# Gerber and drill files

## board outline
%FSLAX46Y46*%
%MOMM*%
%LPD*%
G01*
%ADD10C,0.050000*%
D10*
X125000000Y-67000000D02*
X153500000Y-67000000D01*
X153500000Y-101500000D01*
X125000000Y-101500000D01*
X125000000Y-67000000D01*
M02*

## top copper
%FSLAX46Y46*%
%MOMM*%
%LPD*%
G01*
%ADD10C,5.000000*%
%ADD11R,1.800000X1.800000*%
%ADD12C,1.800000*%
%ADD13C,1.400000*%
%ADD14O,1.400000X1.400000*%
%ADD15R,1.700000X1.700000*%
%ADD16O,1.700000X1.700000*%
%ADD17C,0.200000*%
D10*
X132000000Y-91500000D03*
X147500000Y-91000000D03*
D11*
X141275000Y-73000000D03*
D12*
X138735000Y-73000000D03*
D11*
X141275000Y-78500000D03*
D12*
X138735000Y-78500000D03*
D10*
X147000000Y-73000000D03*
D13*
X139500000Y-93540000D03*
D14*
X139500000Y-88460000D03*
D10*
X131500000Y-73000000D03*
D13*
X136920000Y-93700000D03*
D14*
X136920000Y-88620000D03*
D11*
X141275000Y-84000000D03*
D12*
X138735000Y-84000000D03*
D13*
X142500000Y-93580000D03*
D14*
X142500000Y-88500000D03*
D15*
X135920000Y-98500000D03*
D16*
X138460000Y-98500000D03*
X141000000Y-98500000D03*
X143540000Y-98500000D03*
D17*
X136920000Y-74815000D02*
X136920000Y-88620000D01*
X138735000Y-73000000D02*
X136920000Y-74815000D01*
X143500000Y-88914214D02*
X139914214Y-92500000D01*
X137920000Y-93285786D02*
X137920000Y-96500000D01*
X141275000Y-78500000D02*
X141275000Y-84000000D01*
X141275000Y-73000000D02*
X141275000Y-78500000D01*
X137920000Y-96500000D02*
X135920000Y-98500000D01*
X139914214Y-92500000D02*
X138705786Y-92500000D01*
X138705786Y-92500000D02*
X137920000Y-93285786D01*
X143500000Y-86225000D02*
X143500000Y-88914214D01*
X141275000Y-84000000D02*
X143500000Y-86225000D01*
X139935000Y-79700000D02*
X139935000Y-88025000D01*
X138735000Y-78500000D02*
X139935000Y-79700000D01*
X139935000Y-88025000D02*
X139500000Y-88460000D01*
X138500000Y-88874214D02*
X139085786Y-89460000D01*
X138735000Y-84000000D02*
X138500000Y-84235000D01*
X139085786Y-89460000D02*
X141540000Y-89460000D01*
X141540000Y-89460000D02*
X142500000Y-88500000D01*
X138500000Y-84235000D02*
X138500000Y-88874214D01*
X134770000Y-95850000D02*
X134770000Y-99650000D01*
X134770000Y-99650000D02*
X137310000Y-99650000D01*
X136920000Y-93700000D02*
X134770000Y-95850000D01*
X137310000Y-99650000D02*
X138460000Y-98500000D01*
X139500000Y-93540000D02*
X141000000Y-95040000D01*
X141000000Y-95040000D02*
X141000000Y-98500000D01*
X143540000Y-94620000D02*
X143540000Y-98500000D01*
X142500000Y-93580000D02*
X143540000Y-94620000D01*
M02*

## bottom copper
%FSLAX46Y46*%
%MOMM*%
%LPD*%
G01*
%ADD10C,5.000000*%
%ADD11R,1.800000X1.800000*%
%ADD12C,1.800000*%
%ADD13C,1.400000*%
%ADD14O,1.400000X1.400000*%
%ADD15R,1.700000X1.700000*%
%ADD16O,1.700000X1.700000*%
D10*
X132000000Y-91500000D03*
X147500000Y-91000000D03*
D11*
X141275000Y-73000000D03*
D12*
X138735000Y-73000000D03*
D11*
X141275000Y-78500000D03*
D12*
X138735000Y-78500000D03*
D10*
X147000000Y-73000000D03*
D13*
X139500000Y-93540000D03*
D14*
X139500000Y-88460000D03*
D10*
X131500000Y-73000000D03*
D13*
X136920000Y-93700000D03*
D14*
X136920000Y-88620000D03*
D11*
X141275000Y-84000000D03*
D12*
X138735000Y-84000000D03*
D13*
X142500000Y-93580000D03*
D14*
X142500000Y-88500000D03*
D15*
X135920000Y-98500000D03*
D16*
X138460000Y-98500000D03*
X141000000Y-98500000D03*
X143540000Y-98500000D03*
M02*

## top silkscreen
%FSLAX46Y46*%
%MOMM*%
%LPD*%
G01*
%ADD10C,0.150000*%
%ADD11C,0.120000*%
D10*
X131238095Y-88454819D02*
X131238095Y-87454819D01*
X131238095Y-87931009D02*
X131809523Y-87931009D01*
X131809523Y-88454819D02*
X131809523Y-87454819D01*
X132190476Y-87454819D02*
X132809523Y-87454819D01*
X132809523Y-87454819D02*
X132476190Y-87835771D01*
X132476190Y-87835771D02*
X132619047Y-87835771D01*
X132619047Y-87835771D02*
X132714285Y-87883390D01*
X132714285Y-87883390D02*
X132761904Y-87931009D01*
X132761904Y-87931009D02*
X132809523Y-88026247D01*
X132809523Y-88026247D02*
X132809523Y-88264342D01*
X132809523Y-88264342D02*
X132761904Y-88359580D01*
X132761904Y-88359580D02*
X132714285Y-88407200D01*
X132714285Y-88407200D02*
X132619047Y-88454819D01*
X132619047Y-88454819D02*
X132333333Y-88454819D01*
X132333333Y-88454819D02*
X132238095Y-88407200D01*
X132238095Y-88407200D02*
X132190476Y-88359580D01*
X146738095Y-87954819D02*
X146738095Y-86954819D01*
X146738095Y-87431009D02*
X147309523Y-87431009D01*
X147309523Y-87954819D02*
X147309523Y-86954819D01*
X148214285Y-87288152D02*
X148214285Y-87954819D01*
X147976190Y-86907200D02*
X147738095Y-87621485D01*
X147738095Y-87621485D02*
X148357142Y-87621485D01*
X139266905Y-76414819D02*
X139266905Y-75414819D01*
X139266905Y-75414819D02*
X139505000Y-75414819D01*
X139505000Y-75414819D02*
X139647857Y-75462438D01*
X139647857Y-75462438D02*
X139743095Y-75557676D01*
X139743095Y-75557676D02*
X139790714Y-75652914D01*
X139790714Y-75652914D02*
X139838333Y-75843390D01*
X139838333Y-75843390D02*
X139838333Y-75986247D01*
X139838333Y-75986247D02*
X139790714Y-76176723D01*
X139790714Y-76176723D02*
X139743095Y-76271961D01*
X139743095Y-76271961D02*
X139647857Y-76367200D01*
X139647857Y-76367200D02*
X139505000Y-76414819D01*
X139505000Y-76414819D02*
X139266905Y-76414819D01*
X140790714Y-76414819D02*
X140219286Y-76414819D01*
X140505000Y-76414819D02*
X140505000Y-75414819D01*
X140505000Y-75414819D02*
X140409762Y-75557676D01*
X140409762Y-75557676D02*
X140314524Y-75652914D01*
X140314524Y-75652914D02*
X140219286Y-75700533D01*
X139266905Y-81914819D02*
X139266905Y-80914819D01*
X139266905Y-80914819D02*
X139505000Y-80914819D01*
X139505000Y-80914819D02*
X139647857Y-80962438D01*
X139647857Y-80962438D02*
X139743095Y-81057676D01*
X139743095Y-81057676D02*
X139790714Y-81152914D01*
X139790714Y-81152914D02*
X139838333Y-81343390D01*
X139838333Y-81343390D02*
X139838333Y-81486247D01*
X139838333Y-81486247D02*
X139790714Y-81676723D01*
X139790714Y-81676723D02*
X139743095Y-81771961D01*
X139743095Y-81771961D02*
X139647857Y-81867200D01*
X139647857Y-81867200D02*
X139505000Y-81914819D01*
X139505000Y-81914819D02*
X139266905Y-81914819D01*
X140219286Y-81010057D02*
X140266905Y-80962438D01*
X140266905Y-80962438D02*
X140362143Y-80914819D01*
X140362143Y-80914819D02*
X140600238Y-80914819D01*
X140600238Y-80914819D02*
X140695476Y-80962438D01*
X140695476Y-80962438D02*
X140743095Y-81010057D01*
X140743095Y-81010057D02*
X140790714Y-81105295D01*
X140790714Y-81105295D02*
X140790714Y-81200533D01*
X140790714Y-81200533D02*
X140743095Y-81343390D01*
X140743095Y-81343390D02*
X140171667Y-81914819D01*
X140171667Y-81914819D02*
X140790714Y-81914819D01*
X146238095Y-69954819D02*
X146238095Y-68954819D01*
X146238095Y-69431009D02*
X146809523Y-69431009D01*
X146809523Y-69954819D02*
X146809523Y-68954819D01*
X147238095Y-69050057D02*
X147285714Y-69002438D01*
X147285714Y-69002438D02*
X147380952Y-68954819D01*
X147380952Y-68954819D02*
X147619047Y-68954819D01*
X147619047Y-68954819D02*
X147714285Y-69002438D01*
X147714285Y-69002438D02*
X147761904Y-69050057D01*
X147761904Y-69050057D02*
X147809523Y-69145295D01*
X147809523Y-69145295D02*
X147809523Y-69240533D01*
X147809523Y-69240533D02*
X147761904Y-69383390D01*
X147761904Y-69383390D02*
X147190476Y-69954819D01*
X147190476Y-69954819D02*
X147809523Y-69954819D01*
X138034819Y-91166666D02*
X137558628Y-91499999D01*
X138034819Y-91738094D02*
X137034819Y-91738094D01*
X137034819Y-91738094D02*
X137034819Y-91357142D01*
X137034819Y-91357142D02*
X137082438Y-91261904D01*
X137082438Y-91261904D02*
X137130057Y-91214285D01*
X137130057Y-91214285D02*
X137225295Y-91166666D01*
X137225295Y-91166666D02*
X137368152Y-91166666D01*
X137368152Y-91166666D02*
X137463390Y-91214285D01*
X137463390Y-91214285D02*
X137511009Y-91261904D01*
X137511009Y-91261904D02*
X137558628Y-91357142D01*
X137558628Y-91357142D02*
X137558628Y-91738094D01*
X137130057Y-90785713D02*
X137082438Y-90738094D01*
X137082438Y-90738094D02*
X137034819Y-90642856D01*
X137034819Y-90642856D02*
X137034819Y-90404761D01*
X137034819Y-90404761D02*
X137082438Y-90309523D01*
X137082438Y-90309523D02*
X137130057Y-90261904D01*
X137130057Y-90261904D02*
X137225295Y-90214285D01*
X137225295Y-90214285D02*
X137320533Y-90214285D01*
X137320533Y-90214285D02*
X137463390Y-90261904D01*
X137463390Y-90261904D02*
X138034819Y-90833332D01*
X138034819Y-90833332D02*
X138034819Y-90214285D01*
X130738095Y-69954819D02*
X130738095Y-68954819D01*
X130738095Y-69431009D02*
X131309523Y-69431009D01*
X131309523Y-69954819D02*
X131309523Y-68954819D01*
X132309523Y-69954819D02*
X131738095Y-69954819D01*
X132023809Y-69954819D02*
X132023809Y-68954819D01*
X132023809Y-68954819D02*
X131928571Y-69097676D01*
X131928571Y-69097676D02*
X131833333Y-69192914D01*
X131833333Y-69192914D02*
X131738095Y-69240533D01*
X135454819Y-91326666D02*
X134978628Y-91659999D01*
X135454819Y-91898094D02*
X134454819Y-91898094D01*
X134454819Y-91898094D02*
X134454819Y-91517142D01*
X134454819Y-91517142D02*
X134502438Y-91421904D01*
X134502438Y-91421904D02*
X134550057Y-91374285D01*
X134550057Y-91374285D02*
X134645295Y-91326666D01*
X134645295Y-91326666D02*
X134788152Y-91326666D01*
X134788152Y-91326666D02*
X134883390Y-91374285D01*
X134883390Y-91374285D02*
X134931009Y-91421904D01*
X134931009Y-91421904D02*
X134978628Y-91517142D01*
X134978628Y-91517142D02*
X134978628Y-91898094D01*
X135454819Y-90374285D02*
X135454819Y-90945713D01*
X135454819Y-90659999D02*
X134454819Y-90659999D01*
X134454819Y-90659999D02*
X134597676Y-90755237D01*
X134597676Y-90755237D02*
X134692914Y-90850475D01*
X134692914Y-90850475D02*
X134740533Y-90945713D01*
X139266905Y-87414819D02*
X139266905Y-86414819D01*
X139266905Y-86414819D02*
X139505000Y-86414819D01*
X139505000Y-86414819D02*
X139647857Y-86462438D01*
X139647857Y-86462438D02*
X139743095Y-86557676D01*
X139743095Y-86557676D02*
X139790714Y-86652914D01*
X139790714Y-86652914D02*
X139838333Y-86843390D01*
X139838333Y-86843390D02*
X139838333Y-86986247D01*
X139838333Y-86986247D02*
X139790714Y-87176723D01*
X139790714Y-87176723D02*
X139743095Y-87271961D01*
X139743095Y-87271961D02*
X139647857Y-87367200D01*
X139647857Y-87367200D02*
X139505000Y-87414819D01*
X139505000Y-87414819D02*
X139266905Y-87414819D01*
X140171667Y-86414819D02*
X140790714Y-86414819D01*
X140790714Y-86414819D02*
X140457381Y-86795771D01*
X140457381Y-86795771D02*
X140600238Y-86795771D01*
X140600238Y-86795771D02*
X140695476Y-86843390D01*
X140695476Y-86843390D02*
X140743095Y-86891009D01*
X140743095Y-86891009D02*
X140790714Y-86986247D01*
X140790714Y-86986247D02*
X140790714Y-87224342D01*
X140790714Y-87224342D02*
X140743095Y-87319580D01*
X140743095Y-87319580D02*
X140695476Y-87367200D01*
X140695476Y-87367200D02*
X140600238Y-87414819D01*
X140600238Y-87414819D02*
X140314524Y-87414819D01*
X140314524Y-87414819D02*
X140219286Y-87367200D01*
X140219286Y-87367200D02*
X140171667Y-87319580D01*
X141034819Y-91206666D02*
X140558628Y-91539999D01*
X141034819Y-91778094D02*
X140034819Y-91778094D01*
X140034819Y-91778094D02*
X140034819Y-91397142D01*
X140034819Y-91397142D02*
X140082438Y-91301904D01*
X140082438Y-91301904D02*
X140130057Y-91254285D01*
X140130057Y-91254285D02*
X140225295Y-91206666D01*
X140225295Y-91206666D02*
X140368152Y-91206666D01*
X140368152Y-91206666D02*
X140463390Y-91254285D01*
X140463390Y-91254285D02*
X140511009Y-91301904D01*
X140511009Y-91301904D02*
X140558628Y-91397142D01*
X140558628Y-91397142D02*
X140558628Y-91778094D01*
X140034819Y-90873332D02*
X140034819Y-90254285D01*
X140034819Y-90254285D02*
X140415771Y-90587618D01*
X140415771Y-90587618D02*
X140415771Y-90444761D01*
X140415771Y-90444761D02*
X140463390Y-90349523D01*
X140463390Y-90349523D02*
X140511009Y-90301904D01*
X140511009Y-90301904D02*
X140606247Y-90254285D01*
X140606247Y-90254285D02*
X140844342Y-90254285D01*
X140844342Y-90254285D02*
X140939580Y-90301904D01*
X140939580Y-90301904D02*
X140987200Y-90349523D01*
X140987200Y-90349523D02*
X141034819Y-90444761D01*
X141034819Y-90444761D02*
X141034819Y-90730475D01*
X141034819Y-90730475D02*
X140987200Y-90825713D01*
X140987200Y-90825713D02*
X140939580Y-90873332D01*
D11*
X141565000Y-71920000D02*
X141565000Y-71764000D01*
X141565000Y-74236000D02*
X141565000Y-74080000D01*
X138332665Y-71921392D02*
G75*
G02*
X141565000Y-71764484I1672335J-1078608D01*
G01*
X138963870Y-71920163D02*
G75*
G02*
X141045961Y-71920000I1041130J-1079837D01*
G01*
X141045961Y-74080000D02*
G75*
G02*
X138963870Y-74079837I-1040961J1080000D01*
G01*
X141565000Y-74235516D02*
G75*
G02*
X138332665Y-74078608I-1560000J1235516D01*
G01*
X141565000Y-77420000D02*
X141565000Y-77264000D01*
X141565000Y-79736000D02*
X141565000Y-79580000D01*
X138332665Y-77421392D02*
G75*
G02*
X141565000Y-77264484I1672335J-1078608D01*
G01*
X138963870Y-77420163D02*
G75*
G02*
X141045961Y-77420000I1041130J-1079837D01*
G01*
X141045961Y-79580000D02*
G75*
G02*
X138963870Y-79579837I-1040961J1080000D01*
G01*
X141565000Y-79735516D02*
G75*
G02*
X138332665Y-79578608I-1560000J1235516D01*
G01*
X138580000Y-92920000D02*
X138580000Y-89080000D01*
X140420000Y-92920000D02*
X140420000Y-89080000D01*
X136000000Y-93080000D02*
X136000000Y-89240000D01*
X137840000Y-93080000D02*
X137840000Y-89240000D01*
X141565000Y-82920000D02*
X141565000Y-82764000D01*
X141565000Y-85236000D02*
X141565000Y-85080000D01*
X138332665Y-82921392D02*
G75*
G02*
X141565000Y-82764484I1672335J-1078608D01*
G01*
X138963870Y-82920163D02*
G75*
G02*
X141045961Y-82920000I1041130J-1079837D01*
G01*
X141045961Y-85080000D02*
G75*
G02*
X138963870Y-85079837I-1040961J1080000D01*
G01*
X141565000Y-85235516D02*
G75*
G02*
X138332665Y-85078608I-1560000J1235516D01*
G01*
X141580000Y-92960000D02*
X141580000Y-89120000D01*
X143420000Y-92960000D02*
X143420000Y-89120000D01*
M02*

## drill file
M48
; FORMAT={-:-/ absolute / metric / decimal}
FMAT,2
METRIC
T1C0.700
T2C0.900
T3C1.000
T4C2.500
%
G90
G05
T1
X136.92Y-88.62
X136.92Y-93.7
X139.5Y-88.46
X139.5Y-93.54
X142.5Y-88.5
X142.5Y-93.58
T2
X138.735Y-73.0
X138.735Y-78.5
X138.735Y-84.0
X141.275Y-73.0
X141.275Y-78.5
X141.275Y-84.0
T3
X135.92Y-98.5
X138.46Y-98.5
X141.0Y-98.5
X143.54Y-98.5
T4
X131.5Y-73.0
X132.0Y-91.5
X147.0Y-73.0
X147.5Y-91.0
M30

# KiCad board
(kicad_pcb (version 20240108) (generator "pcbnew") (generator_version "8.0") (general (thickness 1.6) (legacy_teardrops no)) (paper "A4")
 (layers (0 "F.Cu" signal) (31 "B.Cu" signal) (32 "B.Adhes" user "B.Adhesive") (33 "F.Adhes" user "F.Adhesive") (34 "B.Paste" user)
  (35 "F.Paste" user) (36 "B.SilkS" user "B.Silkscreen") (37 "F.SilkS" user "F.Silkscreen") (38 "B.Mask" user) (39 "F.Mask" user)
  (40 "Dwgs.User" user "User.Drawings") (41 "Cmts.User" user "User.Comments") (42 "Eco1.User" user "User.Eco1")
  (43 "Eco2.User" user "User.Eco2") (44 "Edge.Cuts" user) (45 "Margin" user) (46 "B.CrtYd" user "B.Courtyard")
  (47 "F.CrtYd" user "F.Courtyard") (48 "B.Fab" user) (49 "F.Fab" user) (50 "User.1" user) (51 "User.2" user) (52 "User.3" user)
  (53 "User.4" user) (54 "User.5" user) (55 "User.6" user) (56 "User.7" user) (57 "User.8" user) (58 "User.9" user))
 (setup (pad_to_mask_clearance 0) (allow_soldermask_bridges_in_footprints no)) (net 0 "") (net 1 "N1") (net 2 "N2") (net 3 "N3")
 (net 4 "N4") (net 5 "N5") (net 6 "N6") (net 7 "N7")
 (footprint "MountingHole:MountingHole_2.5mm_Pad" (layer "F.Cu") (at 132 91.5)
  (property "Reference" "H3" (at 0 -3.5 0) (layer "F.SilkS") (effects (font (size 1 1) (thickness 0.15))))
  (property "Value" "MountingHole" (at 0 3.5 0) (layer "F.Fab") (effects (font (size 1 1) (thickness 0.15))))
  (pad "1" thru_hole circle (at 0 0) (size 5 5) (drill 2.5) (layers "*.Cu" "*.Mask") (remove_unused_layers no)))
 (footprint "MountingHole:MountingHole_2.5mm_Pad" (layer "F.Cu") (at 147.5 91)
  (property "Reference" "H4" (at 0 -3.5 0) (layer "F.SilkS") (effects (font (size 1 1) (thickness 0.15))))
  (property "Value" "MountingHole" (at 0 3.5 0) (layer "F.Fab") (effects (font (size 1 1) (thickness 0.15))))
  (pad "1" thru_hole circle (at 0 0) (size 5 5) (drill 2.5) (layers "*.Cu" "*.Mask") (remove_unused_layers no)))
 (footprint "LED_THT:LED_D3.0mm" (layer "F.Cu") (at 141.275 73 180)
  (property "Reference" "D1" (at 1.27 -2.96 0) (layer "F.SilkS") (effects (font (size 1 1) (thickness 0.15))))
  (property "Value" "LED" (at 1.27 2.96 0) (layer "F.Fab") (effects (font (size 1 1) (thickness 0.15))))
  (fp_line (start -0.29 1.08) (end -0.29 1.236) (stroke (width 0.12) (type solid)) (layer "F.SilkS"))
  (fp_line (start -0.29 -1.236) (end -0.29 -1.08) (stroke (width 0.12) (type solid)) (layer "F.SilkS"))
  (fp_arc (start 2.942335 1.078608) (mid 1.366487 1.987659) (end -0.29 1.235516) (stroke (width 0.12) (type solid)) (layer "F.SilkS"))
  (fp_arc (start 2.31113 1.079837) (mid 1.270117 1.5) (end 0.229039 1.08) (stroke (width 0.12) (type solid)) (layer "F.SilkS"))
  (fp_arc (start 0.229039 -1.08) (mid 1.270117 -1.5) (end 2.31113 -1.079837) (stroke (width 0.12) (type solid)) (layer "F.SilkS"))
  (fp_arc (start -0.29 -1.235516) (mid 1.366487 -1.987659) (end 2.942335 -1.078608) (stroke (width 0.12) (type solid)) (layer "F.SilkS"))
  (pad "1" thru_hole rect (at 0 0 180) (size 1.8 1.8) (drill 0.9) (layers "*.Cu" "*.Mask") (remove_unused_layers no) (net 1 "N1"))
  (pad "2" thru_hole circle (at 2.54 0 180) (size 1.8 1.8) (drill 0.9) (layers "*.Cu" "*.Mask") (remove_unused_layers no) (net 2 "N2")))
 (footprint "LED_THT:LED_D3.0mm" (layer "F.Cu") (at 141.275 78.5 180)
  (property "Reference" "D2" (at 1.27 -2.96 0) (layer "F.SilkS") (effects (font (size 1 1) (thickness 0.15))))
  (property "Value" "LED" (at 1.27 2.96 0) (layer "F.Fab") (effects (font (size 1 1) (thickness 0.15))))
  (fp_line (start -0.29 1.08) (end -0.29 1.236) (stroke (width 0.12) (type solid)) (layer "F.SilkS"))
  (fp_line (start -0.29 -1.236) (end -0.29 -1.08) (stroke (width 0.12) (type solid)) (layer "F.SilkS"))
  (fp_arc (start 2.942335 1.078608) (mid 1.366487 1.987659) (end -0.29 1.235516) (stroke (width 0.12) (type solid)) (layer "F.SilkS"))
  (fp_arc (start 2.31113 1.079837) (mid 1.270117 1.5) (end 0.229039 1.08) (stroke (width 0.12) (type solid)) (layer "F.SilkS"))
  (fp_arc (start 0.229039 -1.08) (mid 1.270117 -1.5) (end 2.31113 -1.079837) (stroke (width 0.12) (type solid)) (layer "F.SilkS"))
  (fp_arc (start -0.29 -1.235516) (mid 1.366487 -1.987659) (end 2.942335 -1.078608) (stroke (width 0.12) (type solid)) (layer "F.SilkS"))
  (pad "1" thru_hole rect (at 0 0 180) (size 1.8 1.8) (drill 0.9) (layers "*.Cu" "*.Mask") (remove_unused_layers no) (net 1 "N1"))
  (pad "2" thru_hole circle (at 2.54 0 180) (size 1.8 1.8) (drill 0.9) (layers "*.Cu" "*.Mask") (remove_unused_layers no) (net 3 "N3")))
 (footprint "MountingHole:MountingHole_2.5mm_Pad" (layer "F.Cu") (at 147 73)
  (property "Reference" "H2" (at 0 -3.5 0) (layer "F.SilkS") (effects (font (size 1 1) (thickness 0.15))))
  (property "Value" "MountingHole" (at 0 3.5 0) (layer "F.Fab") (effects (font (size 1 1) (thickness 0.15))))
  (pad "1" thru_hole circle (at 0 0) (size 5 5) (drill 2.5) (layers "*.Cu" "*.Mask") (remove_unused_layers no)))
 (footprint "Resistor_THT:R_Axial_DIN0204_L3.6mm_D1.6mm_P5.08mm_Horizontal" (layer "F.Cu") (at 139.5 93.54 90)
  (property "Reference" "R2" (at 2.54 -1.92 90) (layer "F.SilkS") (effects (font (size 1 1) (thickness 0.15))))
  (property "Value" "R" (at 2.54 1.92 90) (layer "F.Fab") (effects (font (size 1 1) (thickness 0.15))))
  (fp_line (start 0.62 -0.92) (end 4.46 -0.92) (stroke (width 0.12) (type solid)) (layer "F.SilkS"))
  (fp_line (start 0.62 0.92) (end 4.46 0.92) (stroke (width 0.12) (type solid)) (layer "F.SilkS"))
  (pad "1" thru_hole circle (at 0 0 90) (size 1.4 1.4) (drill 0.7) (layers "*.Cu" "*.Mask") (remove_unused_layers no) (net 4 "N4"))
  (pad "2" thru_hole oval (at 5.08 0 90) (size 1.4 1.4) (drill 0.7) (layers "*.Cu" "*.Mask") (remove_unused_layers no) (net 3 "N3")))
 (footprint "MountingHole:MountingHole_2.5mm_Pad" (layer "F.Cu") (at 131.5 73)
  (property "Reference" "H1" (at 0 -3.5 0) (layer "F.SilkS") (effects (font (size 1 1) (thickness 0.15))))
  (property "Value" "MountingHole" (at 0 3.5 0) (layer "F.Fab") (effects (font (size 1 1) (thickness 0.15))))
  (pad "1" thru_hole circle (at 0 0) (size 5 5) (drill 2.5) (layers "*.Cu" "*.Mask") (remove_unused_layers no)))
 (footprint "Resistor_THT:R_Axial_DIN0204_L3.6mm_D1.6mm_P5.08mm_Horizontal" (layer "F.Cu") (at 136.92 93.7 90)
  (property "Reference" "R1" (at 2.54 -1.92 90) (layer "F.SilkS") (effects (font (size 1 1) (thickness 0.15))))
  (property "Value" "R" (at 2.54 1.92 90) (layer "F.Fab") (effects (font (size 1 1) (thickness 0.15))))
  (fp_line (start 0.62 -0.92) (end 4.46 -0.92) (stroke (width 0.12) (type solid)) (layer "F.SilkS"))
  (fp_line (start 0.62 0.92) (end 4.46 0.92) (stroke (width 0.12) (type solid)) (layer "F.SilkS"))
  (pad "1" thru_hole circle (at 0 0 90) (size 1.4 1.4) (drill 0.7) (layers "*.Cu" "*.Mask") (remove_unused_layers no) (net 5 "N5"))
  (pad "2" thru_hole oval (at 5.08 0 90) (size 1.4 1.4) (drill 0.7) (layers "*.Cu" "*.Mask") (remove_unused_layers no) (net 2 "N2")))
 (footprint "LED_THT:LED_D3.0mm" (layer "F.Cu") (at 141.275 84 180)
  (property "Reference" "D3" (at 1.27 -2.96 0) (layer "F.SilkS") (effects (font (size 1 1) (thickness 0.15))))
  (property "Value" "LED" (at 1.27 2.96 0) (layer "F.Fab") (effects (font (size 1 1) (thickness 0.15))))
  (fp_line (start -0.29 1.08) (end -0.29 1.236) (stroke (width 0.12) (type solid)) (layer "F.SilkS"))
  (fp_line (start -0.29 -1.236) (end -0.29 -1.08) (stroke (width 0.12) (type solid)) (layer "F.SilkS"))
  (fp_arc (start 2.942335 1.078608) (mid 1.366487 1.987659) (end -0.29 1.235516) (stroke (width 0.12) (type solid)) (layer "F.SilkS"))
  (fp_arc (start 2.31113 1.079837) (mid 1.270117 1.5) (end 0.229039 1.08) (stroke (width 0.12) (type solid)) (layer "F.SilkS"))
  (fp_arc (start 0.229039 -1.08) (mid 1.270117 -1.5) (end 2.31113 -1.079837) (stroke (width 0.12) (type solid)) (layer "F.SilkS"))
  (fp_arc (start -0.29 -1.235516) (mid 1.366487 -1.987659) (end 2.942335 -1.078608) (stroke (width 0.12) (type solid)) (layer "F.SilkS"))
  (pad "1" thru_hole rect (at 0 0 180) (size 1.8 1.8) (drill 0.9) (layers "*.Cu" "*.Mask") (remove_unused_layers no) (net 1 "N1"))
  (pad "2" thru_hole circle (at 2.54 0 180) (size 1.8 1.8) (drill 0.9) (layers "*.Cu" "*.Mask") (remove_unused_layers no) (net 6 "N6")))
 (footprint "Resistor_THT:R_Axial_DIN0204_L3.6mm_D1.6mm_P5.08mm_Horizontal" (layer "F.Cu") (at 142.5 93.58 90)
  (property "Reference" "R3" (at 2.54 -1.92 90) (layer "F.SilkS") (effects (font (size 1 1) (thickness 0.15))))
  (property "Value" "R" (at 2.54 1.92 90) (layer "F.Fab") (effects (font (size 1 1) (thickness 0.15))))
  (fp_line (start 0.62 -0.92) (end 4.46 -0.92) (stroke (width 0.12) (type solid)) (layer "F.SilkS"))
  (fp_line (start 0.62 0.92) (end 4.46 0.92) (stroke (width 0.12) (type solid)) (layer "F.SilkS"))
  (pad "1" thru_hole circle (at 0 0 90) (size 1.4 1.4) (drill 0.7) (layers "*.Cu" "*.Mask") (remove_unused_layers no) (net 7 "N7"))
  (pad "2" thru_hole oval (at 5.08 0 90) (size 1.4 1.4) (drill 0.7) (layers "*.Cu" "*.Mask") (remove_unused_layers no) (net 6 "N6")))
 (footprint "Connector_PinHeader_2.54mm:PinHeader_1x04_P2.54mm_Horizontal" (layer "B.Cu") (at 135.92 98.5 -90)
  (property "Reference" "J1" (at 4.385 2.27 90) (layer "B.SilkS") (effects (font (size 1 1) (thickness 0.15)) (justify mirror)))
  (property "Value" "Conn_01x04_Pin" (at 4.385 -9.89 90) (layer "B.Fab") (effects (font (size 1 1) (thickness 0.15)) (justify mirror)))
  (pad "1" thru_hole rect (at 0 0 270) (size 1.7 1.7) (drill 1) (layers "*.Cu" "*.Mask") (remove_unused_layers no) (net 1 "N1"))
  (pad "2" thru_hole oval (at 0 -2.54 270) (size 1.7 1.7) (drill 1) (layers "*.Cu" "*.Mask") (remove_unused_layers no) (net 5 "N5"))
  (pad "3" thru_hole oval (at 0 -5.08 270) (size 1.7 1.7) (drill 1) (layers "*.Cu" "*.Mask") (remove_unused_layers no) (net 4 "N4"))
  (pad "4" thru_hole oval (at 0 -7.62 270) (size 1.7 1.7) (drill 1) (layers "*.Cu" "*.Mask") (remove_unused_layers no) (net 7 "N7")))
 (gr_rect (start 125 67) (end 153.5 101.5) (stroke (width 0.05) (type default)) (fill none) (layer "Edge.Cuts"))
 (segment (start 136.92 74.815) (end 136.92 88.62) (width 0.2) (layer "F.Cu") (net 2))
 (segment (start 138.735 73) (end 136.92 74.815) (width 0.2) (layer "F.Cu") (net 2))
 (segment (start 143.5 88.914214) (end 139.914214 92.5) (width 0.2) (layer "F.Cu") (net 1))
 (segment (start 137.92 93.285786) (end 137.92 96.5) (width 0.2) (layer "F.Cu") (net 1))
 (segment (start 141.275 78.5) (end 141.275 84) (width 0.2) (layer "F.Cu") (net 1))
 (segment (start 141.275 73) (end 141.275 78.5) (width 0.2) (layer "F.Cu") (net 1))
 (segment (start 137.92 96.5) (end 135.92 98.5) (width 0.2) (layer "F.Cu") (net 1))
 (segment (start 139.914214 92.5) (end 138.705786 92.5) (width 0.2) (layer "F.Cu") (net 1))
 (segment (start 138.705786 92.5) (end 137.92 93.285786) (width 0.2) (layer "F.Cu") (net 1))
 (segment (start 143.5 86.225) (end 143.5 88.914214) (width 0.2) (layer "F.Cu") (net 1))
 (segment (start 141.275 84) (end 143.5 86.225) (width 0.2) (layer "F.Cu") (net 1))
 (segment (start 139.935 79.7) (end 139.935 88.025) (width 0.2) (layer "F.Cu") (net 3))
 (segment (start 138.735 78.5) (end 139.935 79.7) (width 0.2) (layer "F.Cu") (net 3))
 (segment (start 139.935 88.025) (end 139.5 88.46) (width 0.2) (layer "F.Cu") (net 3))
 (segment (start 138.5 88.874214) (end 139.085786 89.46) (width 0.2) (layer "F.Cu") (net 6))
 (segment (start 138.735 84) (end 138.5 84.235) (width 0.2) (layer "F.Cu") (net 6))
 (segment (start 139.085786 89.46) (end 141.54 89.46) (width 0.2) (layer "F.Cu") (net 6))
 (segment (start 141.54 89.46) (end 142.5 88.5) (width 0.2) (layer "F.Cu") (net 6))
 (segment (start 138.5 84.235) (end 138.5 88.874214) (width 0.2) (layer "F.Cu") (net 6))
 (segment (start 134.77 95.85) (end 134.77 99.65) (width 0.2) (layer "F.Cu") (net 5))
 (segment (start 134.77 99.65) (end 137.31 99.65) (width 0.2) (layer "F.Cu") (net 5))
 (segment (start 136.92 93.7) (end 134.77 95.85) (width 0.2) (layer "F.Cu") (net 5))
 (segment (start 137.31 99.65) (end 138.46 98.5) (width 0.2) (layer "F.Cu") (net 5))
 (segment (start 139.5 93.54) (end 141 95.04) (width 0.2) (layer "F.Cu") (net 4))
 (segment (start 141 95.04) (end 141 98.5) (width 0.2) (layer "F.Cu") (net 4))
 (segment (start 143.54 94.62) (end 143.54 98.5) (width 0.2) (layer "F.Cu") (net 7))
 (segment (start 142.5 93.58) (end 143.54 94.62) (width 0.2) (layer "F.Cu") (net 7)))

